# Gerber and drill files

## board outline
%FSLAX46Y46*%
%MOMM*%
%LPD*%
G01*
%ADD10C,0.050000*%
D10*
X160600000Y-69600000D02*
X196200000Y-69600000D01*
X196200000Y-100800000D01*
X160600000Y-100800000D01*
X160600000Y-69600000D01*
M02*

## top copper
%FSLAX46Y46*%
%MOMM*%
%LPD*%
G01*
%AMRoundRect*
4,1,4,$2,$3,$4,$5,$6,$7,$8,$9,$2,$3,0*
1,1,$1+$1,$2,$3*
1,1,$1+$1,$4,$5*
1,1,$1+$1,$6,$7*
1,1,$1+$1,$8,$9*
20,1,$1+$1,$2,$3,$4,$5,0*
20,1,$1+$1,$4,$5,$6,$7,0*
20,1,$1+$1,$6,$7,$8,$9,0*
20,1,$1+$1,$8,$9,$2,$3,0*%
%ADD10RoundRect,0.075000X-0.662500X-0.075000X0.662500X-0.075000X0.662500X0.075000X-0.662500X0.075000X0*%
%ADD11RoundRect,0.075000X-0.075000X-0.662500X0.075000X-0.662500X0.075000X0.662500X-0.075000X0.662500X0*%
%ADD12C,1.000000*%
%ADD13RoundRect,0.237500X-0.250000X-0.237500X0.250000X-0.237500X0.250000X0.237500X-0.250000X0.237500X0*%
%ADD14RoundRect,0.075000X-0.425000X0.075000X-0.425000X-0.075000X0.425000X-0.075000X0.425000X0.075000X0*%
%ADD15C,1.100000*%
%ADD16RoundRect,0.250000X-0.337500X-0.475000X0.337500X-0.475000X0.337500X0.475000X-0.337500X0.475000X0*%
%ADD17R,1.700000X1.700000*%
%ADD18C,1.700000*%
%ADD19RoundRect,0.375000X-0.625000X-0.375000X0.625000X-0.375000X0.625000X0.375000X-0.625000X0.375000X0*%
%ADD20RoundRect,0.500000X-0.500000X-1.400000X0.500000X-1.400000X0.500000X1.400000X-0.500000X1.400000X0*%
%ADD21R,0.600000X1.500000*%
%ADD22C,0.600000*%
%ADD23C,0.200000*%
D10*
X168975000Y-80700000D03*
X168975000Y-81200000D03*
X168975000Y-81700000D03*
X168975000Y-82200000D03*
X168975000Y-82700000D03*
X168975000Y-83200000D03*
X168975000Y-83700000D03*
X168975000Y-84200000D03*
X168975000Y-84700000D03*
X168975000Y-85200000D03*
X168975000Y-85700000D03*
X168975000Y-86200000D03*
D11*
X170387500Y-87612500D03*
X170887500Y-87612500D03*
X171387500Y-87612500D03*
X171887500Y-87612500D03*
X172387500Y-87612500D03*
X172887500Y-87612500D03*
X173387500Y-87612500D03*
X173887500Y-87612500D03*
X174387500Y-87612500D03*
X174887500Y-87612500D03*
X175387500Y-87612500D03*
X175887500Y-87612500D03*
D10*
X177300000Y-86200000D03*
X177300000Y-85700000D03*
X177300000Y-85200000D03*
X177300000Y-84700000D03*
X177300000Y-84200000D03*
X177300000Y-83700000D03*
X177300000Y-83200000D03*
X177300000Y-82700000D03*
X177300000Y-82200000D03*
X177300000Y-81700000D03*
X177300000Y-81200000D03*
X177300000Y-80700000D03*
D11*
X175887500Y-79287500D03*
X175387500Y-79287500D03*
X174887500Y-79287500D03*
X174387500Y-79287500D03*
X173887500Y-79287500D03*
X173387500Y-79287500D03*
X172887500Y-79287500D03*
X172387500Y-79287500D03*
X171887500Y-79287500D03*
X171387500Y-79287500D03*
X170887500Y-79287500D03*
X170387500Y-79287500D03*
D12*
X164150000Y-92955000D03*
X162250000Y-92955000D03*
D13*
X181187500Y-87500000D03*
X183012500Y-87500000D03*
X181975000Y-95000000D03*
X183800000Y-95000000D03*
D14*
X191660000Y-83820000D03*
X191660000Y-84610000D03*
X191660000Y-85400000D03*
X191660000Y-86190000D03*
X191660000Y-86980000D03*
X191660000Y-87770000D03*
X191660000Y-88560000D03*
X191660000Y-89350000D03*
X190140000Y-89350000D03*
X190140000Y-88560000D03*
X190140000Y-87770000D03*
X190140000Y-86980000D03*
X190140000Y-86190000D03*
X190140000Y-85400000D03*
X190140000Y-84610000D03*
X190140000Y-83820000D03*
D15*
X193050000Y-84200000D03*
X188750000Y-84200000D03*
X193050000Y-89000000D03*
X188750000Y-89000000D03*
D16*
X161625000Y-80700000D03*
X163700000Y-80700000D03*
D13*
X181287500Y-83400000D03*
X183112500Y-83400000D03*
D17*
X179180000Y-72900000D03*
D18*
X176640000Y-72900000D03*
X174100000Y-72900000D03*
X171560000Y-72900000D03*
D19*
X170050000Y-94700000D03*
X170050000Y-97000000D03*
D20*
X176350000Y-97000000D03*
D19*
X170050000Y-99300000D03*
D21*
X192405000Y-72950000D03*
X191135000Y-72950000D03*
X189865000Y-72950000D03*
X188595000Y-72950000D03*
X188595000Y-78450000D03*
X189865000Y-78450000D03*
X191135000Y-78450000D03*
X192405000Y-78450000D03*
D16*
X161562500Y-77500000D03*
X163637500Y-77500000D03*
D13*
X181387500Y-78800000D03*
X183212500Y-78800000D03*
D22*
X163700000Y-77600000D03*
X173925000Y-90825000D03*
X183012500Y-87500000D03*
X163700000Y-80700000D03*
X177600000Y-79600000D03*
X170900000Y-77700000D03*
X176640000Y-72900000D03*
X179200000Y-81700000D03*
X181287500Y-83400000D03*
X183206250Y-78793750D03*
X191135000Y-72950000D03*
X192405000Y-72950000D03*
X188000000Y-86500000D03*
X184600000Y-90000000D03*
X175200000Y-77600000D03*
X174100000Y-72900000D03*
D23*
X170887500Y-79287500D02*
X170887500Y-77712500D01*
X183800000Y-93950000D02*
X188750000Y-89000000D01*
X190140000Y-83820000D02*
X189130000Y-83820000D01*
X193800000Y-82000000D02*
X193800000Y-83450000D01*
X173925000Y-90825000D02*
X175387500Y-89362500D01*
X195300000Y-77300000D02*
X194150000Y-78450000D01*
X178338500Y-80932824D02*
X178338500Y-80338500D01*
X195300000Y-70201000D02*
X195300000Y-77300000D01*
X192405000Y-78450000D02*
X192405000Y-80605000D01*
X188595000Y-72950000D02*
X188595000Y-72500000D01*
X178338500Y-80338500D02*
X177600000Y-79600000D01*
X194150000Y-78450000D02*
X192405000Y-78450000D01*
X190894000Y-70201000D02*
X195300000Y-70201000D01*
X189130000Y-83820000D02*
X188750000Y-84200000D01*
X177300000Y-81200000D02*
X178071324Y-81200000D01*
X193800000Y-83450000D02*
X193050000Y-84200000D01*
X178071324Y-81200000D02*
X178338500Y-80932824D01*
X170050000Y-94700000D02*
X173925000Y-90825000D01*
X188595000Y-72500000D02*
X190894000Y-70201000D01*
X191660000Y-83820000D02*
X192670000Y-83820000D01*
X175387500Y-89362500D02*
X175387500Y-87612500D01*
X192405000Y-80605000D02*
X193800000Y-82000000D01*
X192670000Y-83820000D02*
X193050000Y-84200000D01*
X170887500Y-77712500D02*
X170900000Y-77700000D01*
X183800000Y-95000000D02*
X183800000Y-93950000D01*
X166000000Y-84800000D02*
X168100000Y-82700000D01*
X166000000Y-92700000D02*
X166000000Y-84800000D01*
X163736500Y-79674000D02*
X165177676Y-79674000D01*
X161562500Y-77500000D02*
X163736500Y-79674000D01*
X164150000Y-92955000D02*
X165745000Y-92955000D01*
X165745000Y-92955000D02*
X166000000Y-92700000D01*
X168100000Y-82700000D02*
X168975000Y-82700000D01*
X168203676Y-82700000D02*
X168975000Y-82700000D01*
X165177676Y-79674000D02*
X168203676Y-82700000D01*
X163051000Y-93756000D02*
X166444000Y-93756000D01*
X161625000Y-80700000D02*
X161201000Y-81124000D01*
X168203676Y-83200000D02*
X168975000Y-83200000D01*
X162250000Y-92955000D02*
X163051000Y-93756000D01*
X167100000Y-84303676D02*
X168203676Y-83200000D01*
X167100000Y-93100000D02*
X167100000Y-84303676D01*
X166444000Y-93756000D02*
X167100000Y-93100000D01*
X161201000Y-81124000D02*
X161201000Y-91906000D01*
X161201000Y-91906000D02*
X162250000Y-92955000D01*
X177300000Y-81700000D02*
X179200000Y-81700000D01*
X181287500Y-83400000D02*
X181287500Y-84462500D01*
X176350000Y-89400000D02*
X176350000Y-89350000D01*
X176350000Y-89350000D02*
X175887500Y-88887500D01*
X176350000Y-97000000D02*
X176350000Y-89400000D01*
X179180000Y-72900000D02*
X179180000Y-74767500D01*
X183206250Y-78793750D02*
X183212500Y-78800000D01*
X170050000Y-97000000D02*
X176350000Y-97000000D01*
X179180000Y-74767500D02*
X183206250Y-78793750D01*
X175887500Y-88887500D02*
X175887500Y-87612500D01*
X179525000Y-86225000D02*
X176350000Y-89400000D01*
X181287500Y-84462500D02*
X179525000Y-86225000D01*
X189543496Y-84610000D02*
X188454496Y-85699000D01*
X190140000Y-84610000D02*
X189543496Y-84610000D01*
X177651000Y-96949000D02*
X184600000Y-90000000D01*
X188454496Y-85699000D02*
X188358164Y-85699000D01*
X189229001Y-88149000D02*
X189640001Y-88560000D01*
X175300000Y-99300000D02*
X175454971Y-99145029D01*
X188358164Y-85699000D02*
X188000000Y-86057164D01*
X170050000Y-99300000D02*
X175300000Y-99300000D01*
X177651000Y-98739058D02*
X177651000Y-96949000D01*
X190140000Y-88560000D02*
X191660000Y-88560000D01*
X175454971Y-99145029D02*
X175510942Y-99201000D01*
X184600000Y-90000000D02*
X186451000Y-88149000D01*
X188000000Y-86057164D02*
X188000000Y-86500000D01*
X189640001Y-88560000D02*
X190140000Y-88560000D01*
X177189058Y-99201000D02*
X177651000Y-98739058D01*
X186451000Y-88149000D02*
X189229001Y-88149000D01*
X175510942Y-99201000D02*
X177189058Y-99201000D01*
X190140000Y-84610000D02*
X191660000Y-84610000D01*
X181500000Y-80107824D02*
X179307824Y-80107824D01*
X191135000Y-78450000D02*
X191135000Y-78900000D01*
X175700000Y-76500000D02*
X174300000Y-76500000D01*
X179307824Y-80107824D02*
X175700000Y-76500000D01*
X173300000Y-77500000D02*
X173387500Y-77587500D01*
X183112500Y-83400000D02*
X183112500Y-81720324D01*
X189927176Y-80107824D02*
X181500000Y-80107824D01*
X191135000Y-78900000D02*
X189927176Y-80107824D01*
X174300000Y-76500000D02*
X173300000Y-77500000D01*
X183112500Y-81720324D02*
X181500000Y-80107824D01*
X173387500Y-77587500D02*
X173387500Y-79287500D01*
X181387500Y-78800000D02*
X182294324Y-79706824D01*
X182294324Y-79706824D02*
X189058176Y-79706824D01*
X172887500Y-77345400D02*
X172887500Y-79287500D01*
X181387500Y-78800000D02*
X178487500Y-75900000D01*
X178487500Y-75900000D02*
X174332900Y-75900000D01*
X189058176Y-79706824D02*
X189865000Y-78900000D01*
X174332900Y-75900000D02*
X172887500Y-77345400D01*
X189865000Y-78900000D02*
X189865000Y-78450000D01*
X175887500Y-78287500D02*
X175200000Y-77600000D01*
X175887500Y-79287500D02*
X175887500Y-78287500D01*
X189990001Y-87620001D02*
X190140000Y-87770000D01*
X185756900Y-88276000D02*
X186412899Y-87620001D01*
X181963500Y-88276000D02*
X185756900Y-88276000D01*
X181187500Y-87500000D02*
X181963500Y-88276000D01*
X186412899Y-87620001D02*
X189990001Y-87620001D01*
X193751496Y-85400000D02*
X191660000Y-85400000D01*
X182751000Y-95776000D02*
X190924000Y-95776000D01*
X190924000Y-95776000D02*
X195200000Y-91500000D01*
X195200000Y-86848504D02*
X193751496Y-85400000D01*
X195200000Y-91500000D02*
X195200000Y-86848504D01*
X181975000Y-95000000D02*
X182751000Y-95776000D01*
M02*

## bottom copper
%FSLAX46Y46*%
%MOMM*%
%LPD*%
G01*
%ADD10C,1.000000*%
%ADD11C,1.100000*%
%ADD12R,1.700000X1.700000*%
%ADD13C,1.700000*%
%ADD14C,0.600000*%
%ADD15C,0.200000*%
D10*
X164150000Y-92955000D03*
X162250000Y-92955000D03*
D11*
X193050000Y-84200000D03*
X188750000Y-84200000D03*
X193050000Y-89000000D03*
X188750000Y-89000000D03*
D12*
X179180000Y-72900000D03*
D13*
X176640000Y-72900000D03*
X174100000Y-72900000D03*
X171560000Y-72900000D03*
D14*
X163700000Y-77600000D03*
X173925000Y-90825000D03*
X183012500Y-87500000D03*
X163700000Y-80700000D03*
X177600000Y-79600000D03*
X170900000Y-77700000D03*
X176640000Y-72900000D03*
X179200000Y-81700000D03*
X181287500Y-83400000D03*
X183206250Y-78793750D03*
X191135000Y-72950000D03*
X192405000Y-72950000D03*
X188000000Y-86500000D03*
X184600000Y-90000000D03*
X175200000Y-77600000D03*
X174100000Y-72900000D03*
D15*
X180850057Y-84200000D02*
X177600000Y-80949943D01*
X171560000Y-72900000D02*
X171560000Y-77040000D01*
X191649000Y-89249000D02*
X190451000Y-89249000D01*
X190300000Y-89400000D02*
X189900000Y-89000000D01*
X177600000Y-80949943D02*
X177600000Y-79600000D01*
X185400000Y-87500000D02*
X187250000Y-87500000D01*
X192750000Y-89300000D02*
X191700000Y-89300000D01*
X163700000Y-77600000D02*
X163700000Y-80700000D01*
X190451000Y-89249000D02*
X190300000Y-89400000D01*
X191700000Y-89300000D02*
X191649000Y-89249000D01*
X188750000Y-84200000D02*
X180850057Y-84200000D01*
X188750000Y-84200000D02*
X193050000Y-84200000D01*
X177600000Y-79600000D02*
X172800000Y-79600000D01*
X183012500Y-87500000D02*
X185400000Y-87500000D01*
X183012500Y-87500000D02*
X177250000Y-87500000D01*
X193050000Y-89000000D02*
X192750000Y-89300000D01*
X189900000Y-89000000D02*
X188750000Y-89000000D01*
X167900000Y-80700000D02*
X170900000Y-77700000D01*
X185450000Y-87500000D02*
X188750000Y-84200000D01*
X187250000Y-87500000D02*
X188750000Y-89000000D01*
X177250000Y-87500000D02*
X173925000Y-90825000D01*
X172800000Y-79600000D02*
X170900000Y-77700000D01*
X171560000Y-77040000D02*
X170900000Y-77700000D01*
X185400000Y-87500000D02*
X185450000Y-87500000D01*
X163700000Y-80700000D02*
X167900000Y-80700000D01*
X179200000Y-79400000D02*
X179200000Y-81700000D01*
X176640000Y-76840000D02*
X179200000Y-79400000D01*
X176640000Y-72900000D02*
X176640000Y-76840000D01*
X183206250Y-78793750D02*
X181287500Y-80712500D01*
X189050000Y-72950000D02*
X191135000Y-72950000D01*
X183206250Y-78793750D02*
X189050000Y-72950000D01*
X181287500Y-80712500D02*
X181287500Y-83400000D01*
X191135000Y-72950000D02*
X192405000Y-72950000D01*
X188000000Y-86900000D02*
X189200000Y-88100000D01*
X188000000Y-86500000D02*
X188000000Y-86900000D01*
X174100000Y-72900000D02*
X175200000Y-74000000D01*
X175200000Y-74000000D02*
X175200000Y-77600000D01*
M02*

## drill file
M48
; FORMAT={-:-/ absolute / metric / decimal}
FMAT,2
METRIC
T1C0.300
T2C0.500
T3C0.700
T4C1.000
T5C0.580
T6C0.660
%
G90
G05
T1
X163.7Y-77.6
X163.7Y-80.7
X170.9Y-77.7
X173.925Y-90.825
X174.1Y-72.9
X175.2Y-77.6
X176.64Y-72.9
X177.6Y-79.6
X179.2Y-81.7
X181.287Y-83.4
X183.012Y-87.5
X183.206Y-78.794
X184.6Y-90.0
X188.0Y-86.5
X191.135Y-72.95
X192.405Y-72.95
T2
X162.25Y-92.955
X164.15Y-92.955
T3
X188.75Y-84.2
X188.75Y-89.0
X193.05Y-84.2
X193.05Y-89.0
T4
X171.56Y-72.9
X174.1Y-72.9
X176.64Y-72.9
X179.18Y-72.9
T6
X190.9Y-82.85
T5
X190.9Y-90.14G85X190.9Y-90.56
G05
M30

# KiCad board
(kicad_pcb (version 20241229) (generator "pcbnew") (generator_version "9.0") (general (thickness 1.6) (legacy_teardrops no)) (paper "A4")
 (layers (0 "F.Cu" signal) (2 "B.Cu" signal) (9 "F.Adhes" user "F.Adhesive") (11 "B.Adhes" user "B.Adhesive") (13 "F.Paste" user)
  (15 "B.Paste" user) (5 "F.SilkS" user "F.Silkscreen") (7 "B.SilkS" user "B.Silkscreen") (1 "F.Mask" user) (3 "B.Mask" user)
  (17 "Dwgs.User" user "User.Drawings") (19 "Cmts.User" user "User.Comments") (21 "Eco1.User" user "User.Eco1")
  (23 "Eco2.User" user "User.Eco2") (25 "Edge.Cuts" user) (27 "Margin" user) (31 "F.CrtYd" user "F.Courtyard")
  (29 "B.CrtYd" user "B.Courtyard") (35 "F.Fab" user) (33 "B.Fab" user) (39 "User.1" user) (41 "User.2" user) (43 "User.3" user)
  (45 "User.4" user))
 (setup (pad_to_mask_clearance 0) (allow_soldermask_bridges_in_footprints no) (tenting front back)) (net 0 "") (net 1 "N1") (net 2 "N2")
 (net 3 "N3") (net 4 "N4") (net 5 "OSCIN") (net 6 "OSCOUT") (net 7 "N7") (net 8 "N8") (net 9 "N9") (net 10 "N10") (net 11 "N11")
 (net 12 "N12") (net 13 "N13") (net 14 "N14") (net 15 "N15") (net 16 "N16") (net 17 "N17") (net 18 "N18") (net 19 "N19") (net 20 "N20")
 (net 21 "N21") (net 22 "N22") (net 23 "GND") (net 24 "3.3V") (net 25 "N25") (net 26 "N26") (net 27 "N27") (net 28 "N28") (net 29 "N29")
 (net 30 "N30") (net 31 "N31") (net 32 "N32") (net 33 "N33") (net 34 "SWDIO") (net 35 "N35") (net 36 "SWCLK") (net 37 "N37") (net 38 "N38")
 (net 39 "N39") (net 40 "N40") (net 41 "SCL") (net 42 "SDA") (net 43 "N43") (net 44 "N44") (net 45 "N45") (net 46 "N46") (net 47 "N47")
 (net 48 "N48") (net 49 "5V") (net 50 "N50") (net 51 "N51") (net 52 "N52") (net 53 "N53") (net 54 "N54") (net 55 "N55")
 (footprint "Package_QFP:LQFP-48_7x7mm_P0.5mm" (layer "F.Cu") (at 173.1375 83.45)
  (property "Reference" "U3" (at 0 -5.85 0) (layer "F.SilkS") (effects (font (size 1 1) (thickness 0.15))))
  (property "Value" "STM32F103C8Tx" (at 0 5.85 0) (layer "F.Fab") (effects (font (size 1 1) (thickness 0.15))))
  (pad "1" smd roundrect (at -4.1625 -2.75) (size 1.475 0.3) (layers "F.Cu" "F.Mask" "F.Paste") (roundrect_rratio 0.25) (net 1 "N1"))
  (pad "2" smd roundrect (at -4.1625 -2.25) (size 1.475 0.3) (layers "F.Cu" "F.Mask" "F.Paste") (roundrect_rratio 0.25) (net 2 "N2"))
  (pad "3" smd roundrect (at -4.1625 -1.75) (size 1.475 0.3) (layers "F.Cu" "F.Mask" "F.Paste") (roundrect_rratio 0.25) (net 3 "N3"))
  (pad "4" smd roundrect (at -4.1625 -1.25) (size 1.475 0.3) (layers "F.Cu" "F.Mask" "F.Paste") (roundrect_rratio 0.25) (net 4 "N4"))
  (pad "5" smd roundrect (at -4.1625 -0.75) (size 1.475 0.3) (layers "F.Cu" "F.Mask" "F.Paste") (roundrect_rratio 0.25) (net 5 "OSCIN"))
  (pad "6" smd roundrect (at -4.1625 -0.25) (size 1.475 0.3) (layers "F.Cu" "F.Mask" "F.Paste") (roundrect_rratio 0.25) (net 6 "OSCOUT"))
  (pad "7" smd roundrect (at -4.1625 0.25) (size 1.475 0.3) (layers "F.Cu" "F.Mask" "F.Paste") (roundrect_rratio 0.25) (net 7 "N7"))
  (pad "8" smd roundrect (at -4.1625 0.75) (size 1.475 0.3) (layers "F.Cu" "F.Mask" "F.Paste") (roundrect_rratio 0.25) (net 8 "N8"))
  (pad "9" smd roundrect (at -4.1625 1.25) (size 1.475 0.3) (layers "F.Cu" "F.Mask" "F.Paste") (roundrect_rratio 0.25) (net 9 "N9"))
  (pad "10" smd roundrect (at -4.1625 1.75) (size 1.475 0.3) (layers "F.Cu" "F.Mask" "F.Paste") (roundrect_rratio 0.25) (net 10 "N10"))
  (pad "11" smd roundrect (at -4.1625 2.25) (size 1.475 0.3) (layers "F.Cu" "F.Mask" "F.Paste") (roundrect_rratio 0.25) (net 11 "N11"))
  (pad "12" smd roundrect (at -4.1625 2.75) (size 1.475 0.3) (layers "F.Cu" "F.Mask" "F.Paste") (roundrect_rratio 0.25) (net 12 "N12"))
  (pad "13" smd roundrect (at -2.75 4.1625) (size 0.3 1.475) (layers "F.Cu" "F.Mask" "F.Paste") (roundrect_rratio 0.25) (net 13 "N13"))
  (pad "14" smd roundrect (at -2.25 4.1625) (size 0.3 1.475) (layers "F.Cu" "F.Mask" "F.Paste") (roundrect_rratio 0.25) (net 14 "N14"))
  (pad "15" smd roundrect (at -1.75 4.1625) (size 0.3 1.475) (layers "F.Cu" "F.Mask" "F.Paste") (roundrect_rratio 0.25) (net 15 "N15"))
  (pad "16" smd roundrect (at -1.25 4.1625) (size 0.3 1.475) (layers "F.Cu" "F.Mask" "F.Paste") (roundrect_rratio 0.25) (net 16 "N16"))
  (pad "17" smd roundrect (at -0.75 4.1625) (size 0.3 1.475) (layers "F.Cu" "F.Mask" "F.Paste") (roundrect_rratio 0.25) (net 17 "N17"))
  (pad "18" smd roundrect (at -0.25 4.1625) (size 0.3 1.475) (layers "F.Cu" "F.Mask" "F.Paste") (roundrect_rratio 0.25) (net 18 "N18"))
  (pad "19" smd roundrect (at 0.25 4.1625) (size 0.3 1.475) (layers "F.Cu" "F.Mask" "F.Paste") (roundrect_rratio 0.25) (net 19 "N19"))
  (pad "20" smd roundrect (at 0.75 4.1625) (size 0.3 1.475) (layers "F.Cu" "F.Mask" "F.Paste") (roundrect_rratio 0.25) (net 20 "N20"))
  (pad "21" smd roundrect (at 1.25 4.1625) (size 0.3 1.475) (layers "F.Cu" "F.Mask" "F.Paste") (roundrect_rratio 0.25) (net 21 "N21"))
  (pad "22" smd roundrect (at 1.75 4.1625) (size 0.3 1.475) (layers "F.Cu" "F.Mask" "F.Paste") (roundrect_rratio 0.25) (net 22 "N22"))
  (pad "23" smd roundrect (at 2.25 4.1625) (size 0.3 1.475) (layers "F.Cu" "F.Mask" "F.Paste") (roundrect_rratio 0.25) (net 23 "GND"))
  (pad "24" smd roundrect (at 2.75 4.1625) (size 0.3 1.475) (layers "F.Cu" "F.Mask" "F.Paste") (roundrect_rratio 0.25) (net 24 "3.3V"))
  (pad "25" smd roundrect (at 4.1625 2.75) (size 1.475 0.3) (layers "F.Cu" "F.Mask" "F.Paste") (roundrect_rratio 0.25) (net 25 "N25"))
  (pad "26" smd roundrect (at 4.1625 2.25) (size 1.475 0.3) (layers "F.Cu" "F.Mask" "F.Paste") (roundrect_rratio 0.25) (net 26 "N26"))
  (pad "27" smd roundrect (at 4.1625 1.75) (size 1.475 0.3) (layers "F.Cu" "F.Mask" "F.Paste") (roundrect_rratio 0.25) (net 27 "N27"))
  (pad "28" smd roundrect (at 4.1625 1.25) (size 1.475 0.3) (layers "F.Cu" "F.Mask" "F.Paste") (roundrect_rratio 0.25) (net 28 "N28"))
  (pad "29" smd roundrect (at 4.1625 0.75) (size 1.475 0.3) (layers "F.Cu" "F.Mask" "F.Paste") (roundrect_rratio 0.25) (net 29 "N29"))
  (pad "30" smd roundrect (at 4.1625 0.25) (size 1.475 0.3) (layers "F.Cu" "F.Mask" "F.Paste") (roundrect_rratio 0.25) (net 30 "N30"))
  (pad "31" smd roundrect (at 4.1625 -0.25) (size 1.475 0.3) (layers "F.Cu" "F.Mask" "F.Paste") (roundrect_rratio 0.25) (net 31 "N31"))
  (pad "32" smd roundrect (at 4.1625 -0.75) (size 1.475 0.3) (layers "F.Cu" "F.Mask" "F.Paste") (roundrect_rratio 0.25) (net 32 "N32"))
  (pad "33" smd roundrect (at 4.1625 -1.25) (size 1.475 0.3) (layers "F.Cu" "F.Mask" "F.Paste") (roundrect_rratio 0.25) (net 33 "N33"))
  (pad "34" smd roundrect (at 4.1625 -1.75) (size 1.475 0.3) (layers "F.Cu" "F.Mask" "F.Paste") (roundrect_rratio 0.25) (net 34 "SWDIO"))
  (pad "35" smd roundrect (at 4.1625 -2.25) (size 1.475 0.3) (layers "F.Cu" "F.Mask" "F.Paste") (roundrect_rratio 0.25) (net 23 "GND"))
  (pad "36" smd roundrect (at 4.1625 -2.75) (size 1.475 0.3) (layers "F.Cu" "F.Mask" "F.Paste") (roundrect_rratio 0.25) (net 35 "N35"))
  (pad "37" smd roundrect (at 2.75 -4.1625) (size 0.3 1.475) (layers "F.Cu" "F.Mask" "F.Paste") (roundrect_rratio 0.25) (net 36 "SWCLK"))
  (pad "38" smd roundrect (at 2.25 -4.1625) (size 0.3 1.475) (layers "F.Cu" "F.Mask" "F.Paste") (roundrect_rratio 0.25) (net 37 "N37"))
  (pad "39" smd roundrect (at 1.75 -4.1625) (size 0.3 1.475) (layers "F.Cu" "F.Mask" "F.Paste") (roundrect_rratio 0.25) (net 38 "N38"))
  (pad "40" smd roundrect (at 1.25 -4.1625) (size 0.3 1.475) (layers "F.Cu" "F.Mask" "F.Paste") (roundrect_rratio 0.25) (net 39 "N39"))
  (pad "41" smd roundrect (at 0.75 -4.1625) (size 0.3 1.475) (layers "F.Cu" "F.Mask" "F.Paste") (roundrect_rratio 0.25) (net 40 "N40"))
  (pad "42" smd roundrect (at 0.25 -4.1625) (size 0.3 1.475) (layers "F.Cu" "F.Mask" "F.Paste") (roundrect_rratio 0.25) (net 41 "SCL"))
  (pad "43" smd roundrect (at -0.25 -4.1625) (size 0.3 1.475) (layers "F.Cu" "F.Mask" "F.Paste") (roundrect_rratio 0.25) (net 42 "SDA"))
  (pad "44" smd roundrect (at -0.75 -4.1625) (size 0.3 1.475) (layers "F.Cu" "F.Mask" "F.Paste") (roundrect_rratio 0.25) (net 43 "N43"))
  (pad "45" smd roundrect (at -1.25 -4.1625) (size 0.3 1.475) (layers "F.Cu" "F.Mask" "F.Paste") (roundrect_rratio 0.25) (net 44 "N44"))
  (pad "46" smd roundrect (at -1.75 -4.1625) (size 0.3 1.475) (layers "F.Cu" "F.Mask" "F.Paste") (roundrect_rratio 0.25) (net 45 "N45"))
  (pad "47" smd roundrect (at -2.25 -4.1625) (size 0.3 1.475) (layers "F.Cu" "F.Mask" "F.Paste") (roundrect_rratio 0.25) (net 23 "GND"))
  (pad "48" smd roundrect (at -2.75 -4.1625) (size 0.3 1.475) (layers "F.Cu" "F.Mask" "F.Paste") (roundrect_rratio 0.25) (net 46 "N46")))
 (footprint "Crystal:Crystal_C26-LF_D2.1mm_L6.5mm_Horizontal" (layer "F.Cu") (at 164.15 92.955 180)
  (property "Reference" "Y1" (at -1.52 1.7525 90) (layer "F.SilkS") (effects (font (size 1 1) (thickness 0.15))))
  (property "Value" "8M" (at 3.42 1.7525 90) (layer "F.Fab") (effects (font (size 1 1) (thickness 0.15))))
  (pad "1" thru_hole circle (at 0 0 180) (size 1 1) (drill 0.5) (layers "*.Cu" "*.Mask") (remove_unused_layers no) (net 5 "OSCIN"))
  (pad "2" thru_hole circle (at 1.9 0 180) (size 1 1) (drill 0.5) (layers "*.Cu" "*.Mask") (remove_unused_layers no) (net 6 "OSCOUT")))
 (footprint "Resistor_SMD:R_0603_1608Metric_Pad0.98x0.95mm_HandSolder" (layer "F.Cu") (at 182.1 87.5)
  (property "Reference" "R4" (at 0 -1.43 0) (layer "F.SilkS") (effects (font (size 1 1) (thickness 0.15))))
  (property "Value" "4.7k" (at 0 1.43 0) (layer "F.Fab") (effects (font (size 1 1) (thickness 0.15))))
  (pad "1" smd roundrect (at -0.9125 0) (size 0.975 0.95) (layers "F.Cu" "F.Mask" "F.Paste") (roundrect_rratio 0.25) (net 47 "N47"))
  (pad "2" smd roundrect (at 0.9125 0) (size 0.975 0.95) (layers "F.Cu" "F.Mask" "F.Paste") (roundrect_rratio 0.25) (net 23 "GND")))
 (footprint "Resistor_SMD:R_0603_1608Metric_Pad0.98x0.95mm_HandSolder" (layer "F.Cu") (at 182.8875 95)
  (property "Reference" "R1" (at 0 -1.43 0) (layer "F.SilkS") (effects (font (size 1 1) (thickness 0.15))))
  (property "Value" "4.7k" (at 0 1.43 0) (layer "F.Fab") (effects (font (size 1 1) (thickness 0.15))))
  (pad "1" smd roundrect (at -0.9125 0) (size 0.975 0.95) (layers "F.Cu" "F.Mask" "F.Paste") (roundrect_rratio 0.25) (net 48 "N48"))
  (pad "2" smd roundrect (at 0.9125 0) (size 0.975 0.95) (layers "F.Cu" "F.Mask" "F.Paste") (roundrect_rratio 0.25) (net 23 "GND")))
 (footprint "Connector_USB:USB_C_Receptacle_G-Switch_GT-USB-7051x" (layer "F.Cu") (at 190.9 86.6 -90)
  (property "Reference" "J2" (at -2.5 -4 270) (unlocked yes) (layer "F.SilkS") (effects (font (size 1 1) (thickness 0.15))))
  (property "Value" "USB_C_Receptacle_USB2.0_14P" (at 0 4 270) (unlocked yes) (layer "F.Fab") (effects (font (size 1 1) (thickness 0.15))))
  (pad "" np_thru_hole circle (at -3.75 0 270) (size 0.66 0.66) (drill 0.66) (layers "*.Cu" "*.Mask"))
  (pad "" np_thru_hole oval (at 3.75 0 270) (size 1 0.58) (drill oval 1 0.58) (layers "*.Cu" "*.Mask"))
  (pad "A1" smd roundrect (at -2.78 -0.76 270) (size 0.3 1) (layers "F.Cu" "F.Mask" "F.Paste") (roundrect_rratio 0.25) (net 23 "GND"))
  (pad "A4" smd roundrect (at -1.99 -0.76 270) (size 0.3 1) (layers "F.Cu" "F.Mask" "F.Paste") (roundrect_rratio 0.25) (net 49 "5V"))
  (pad "A5" smd roundrect (at -1.2 -0.76 270) (size 0.3 1) (layers "F.Cu" "F.Mask" "F.Paste") (roundrect_rratio 0.25) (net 48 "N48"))
  (pad "A6" smd roundrect (at -0.41 -0.76 270) (size 0.3 1) (layers "F.Cu" "F.Mask" "F.Paste") (roundrect_rratio 0.25) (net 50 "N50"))
  (pad "A7" smd roundrect (at 0.38 -0.76 270) (size 0.3 1) (layers "F.Cu" "F.Mask" "F.Paste") (roundrect_rratio 0.25) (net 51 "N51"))
  (pad "A8" smd roundrect (at 1.17 -0.76 270) (size 0.3 1) (layers "F.Cu" "F.Mask" "F.Paste") (roundrect_rratio 0.25))
  (pad "A9" smd roundrect (at 1.96 -0.76 270) (size 0.3 1) (layers "F.Cu" "F.Mask" "F.Paste") (roundrect_rratio 0.25) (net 49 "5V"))
  (pad "A12" smd roundrect (at 2.75 -0.76 270) (size 0.3 1) (layers "F.Cu" "F.Mask" "F.Paste") (roundrect_rratio 0.25) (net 23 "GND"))
  (pad "B1" smd roundrect (at 2.75 0.76 270) (size 0.3 1) (layers "F.Cu" "F.Mask" "F.Paste") (roundrect_rratio 0.25) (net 23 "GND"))
  (pad "B4" smd roundrect (at 1.96 0.76 270) (size 0.3 1) (layers "F.Cu" "F.Mask" "F.Paste") (roundrect_rratio 0.25) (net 49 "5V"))
  (pad "B5" smd roundrect (at 1.17 0.76 270) (size 0.3 1) (layers "F.Cu" "F.Mask" "F.Paste") (roundrect_rratio 0.25) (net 47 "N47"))
  (pad "B6" smd roundrect (at 0.38 0.76 270) (size 0.3 1) (layers "F.Cu" "F.Mask" "F.Paste") (roundrect_rratio 0.25) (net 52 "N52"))
  (pad "B7" smd roundrect (at -0.41 0.76 270) (size 0.3 1) (layers "F.Cu" "F.Mask" "F.Paste") (roundrect_rratio 0.25) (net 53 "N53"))
  (pad "B8" smd roundrect (at -1.2 0.76 270) (size 0.3 1) (layers "F.Cu" "F.Mask" "F.Paste") (roundrect_rratio 0.25))
  (pad "B9" smd roundrect (at -1.99 0.76 270) (size 0.3 1) (layers "F.Cu" "F.Mask" "F.Paste") (roundrect_rratio 0.25) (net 49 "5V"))
  (pad "B12" smd roundrect (at -2.78 0.76 270) (size 0.3 1) (layers "F.Cu" "F.Mask" "F.Paste") (roundrect_rratio 0.25) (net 23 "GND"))
  (pad "S1" thru_hole circle (at -2.4 -2.15 270) (size 1.1 1.1) (drill 0.7) (layers "*.Cu" "*.Mask" "F.Paste") (remove_unused_layers no)
   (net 23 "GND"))
  (pad "S1" thru_hole circle (at -2.4 2.15 270) (size 1.1 1.1) (drill 0.7) (layers "*.Cu" "*.Mask" "F.Paste") (remove_unused_layers no)
   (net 23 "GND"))
  (pad "S1" thru_hole circle (at 2.4 -2.15 270) (size 1.1 1.1) (drill 0.7) (layers "*.Cu" "*.Mask" "F.Paste") (remove_unused_layers no)
   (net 23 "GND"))
  (pad "S1" thru_hole circle (at 2.4 2.15 270) (size 1.1 1.1) (drill 0.7) (layers "*.Cu" "*.Mask" "F.Paste") (remove_unused_layers no)
   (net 23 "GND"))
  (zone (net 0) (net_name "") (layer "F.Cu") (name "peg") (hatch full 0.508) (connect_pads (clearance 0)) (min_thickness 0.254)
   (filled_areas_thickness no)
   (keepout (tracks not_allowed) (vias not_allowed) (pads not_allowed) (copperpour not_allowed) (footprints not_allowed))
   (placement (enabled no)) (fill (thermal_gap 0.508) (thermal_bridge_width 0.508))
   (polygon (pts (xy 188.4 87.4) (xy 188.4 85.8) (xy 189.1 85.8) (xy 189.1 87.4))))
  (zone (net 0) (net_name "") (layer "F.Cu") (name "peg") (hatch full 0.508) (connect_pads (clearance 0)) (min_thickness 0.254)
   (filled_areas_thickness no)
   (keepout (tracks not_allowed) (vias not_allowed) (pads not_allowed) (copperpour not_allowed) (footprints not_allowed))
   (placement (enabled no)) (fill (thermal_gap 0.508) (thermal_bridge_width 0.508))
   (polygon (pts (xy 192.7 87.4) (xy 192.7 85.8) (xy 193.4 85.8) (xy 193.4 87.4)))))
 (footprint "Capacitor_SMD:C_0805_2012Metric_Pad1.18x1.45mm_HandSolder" (layer "F.Cu") (at 162.6625 80.7)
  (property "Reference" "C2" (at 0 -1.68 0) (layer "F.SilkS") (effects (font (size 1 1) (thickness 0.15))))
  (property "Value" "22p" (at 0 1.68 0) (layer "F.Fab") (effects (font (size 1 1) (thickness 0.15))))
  (pad "1" smd roundrect (at -1.0375 0) (size 1.175 1.45) (layers "F.Cu" "F.Mask" "F.Paste") (roundrect_rratio 0.212766) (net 6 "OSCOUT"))
  (pad "2" smd roundrect (at 1.0375 0) (size 1.175 1.45) (layers "F.Cu" "F.Mask" "F.Paste") (roundrect_rratio 0.212766) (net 23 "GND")))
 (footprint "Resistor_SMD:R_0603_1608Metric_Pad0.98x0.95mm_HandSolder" (layer "F.Cu") (at 182.2 83.4)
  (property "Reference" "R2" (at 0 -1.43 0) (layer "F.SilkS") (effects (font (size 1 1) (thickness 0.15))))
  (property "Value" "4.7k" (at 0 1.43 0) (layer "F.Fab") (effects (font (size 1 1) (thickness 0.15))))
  (pad "1" smd roundrect (at -0.9125 0) (size 0.975 0.95) (layers "F.Cu" "F.Mask" "F.Paste") (roundrect_rratio 0.25) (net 24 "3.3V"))
  (pad "2" smd roundrect (at 0.9125 0) (size 0.975 0.95) (layers "F.Cu" "F.Mask" "F.Paste") (roundrect_rratio 0.25) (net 41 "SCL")))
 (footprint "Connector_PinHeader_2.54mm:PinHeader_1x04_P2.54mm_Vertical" (layer "F.Cu") (at 179.18 72.9 -90)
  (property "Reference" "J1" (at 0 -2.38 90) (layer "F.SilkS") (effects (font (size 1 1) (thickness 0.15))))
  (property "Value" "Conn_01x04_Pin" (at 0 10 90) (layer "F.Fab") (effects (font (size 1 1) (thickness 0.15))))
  (pad "1" thru_hole rect (at 0 0 270) (size 1.7 1.7) (drill 1) (layers "*.Cu" "*.Mask") (remove_unused_layers no) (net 24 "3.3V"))
  (pad "2" thru_hole circle (at 0 2.54 270) (size 1.7 1.7) (drill 1) (layers "*.Cu" "*.Mask") (remove_unused_layers no) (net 34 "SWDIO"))
  (pad "3" thru_hole circle (at 0 5.08 270) (size 1.7 1.7) (drill 1) (layers "*.Cu" "*.Mask") (remove_unused_layers no) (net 36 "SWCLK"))
  (pad "4" thru_hole circle (at 0 7.62 270) (size 1.7 1.7) (drill 1) (layers "*.Cu" "*.Mask") (remove_unused_layers no) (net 23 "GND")))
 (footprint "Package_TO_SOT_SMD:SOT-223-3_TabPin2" (layer "F.Cu") (at 173.2 97)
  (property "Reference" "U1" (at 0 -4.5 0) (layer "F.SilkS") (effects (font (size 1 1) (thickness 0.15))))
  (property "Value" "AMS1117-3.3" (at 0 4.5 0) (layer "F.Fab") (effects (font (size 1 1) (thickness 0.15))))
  (pad "1" smd roundrect (at -3.15 -2.3) (size 2 1.5) (layers "F.Cu" "F.Mask" "F.Paste") (roundrect_rratio 0.25) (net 23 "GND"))
  (pad "2" smd roundrect (at -3.15 0) (size 2 1.5) (layers "F.Cu" "F.Mask" "F.Paste") (roundrect_rratio 0.25) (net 24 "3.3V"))
  (pad "2" smd roundrect (at 3.15 0) (size 2 3.8) (layers "F.Cu" "F.Mask" "F.Paste") (roundrect_rratio 0.25) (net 24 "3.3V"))
  (pad "3" smd roundrect (at -3.15 2.3) (size 2 1.5) (layers "F.Cu" "F.Mask" "F.Paste") (roundrect_rratio 0.25) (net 49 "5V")))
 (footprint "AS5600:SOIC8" (layer "F.Cu") (at 190.5 75.7 180)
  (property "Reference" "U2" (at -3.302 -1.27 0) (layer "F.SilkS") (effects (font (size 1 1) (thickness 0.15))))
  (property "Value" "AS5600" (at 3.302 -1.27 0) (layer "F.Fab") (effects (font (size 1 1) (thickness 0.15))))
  (pad "1" smd rect (at -1.905 2.75 180) (size 0.6 1.5) (layers "F.Cu" "F.Mask" "F.Paste") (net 24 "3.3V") (solder_mask_margin 0.102))
  (pad "2" smd rect (at -0.635 2.75 180) (size 0.6 1.5) (layers "F.Cu" "F.Mask" "F.Paste") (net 24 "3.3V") (solder_mask_margin 0.102))
  (pad "3" smd rect (at 0.635 2.75 180) (size 0.6 1.5) (layers "F.Cu" "F.Mask" "F.Paste") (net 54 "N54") (solder_mask_margin 0.102))
  (pad "4" smd rect (at 1.905 2.75 180) (size 0.6 1.5) (layers "F.Cu" "F.Mask" "F.Paste") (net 23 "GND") (solder_mask_margin 0.102))
  (pad "5" smd rect (at 1.905 -2.75 180) (size 0.6 1.5) (layers "F.Cu" "F.Mask" "F.Paste") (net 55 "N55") (solder_mask_margin 0.102))
  (pad "6" smd rect (at 0.635 -2.75 180) (size 0.6 1.5) (layers "F.Cu" "F.Mask" "F.Paste") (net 42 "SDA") (solder_mask_margin 0.102))
  (pad "7" smd rect (at -0.635 -2.75 180) (size 0.6 1.5) (layers "F.Cu" "F.Mask" "F.Paste") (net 41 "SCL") (solder_mask_margin 0.102))
  (pad "8" smd rect (at -1.905 -2.75 180) (size 0.6 1.5) (layers "F.Cu" "F.Mask" "F.Paste") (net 23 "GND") (solder_mask_margin 0.102)))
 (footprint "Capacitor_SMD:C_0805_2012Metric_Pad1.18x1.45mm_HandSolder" (layer "F.Cu") (at 162.6 77.5)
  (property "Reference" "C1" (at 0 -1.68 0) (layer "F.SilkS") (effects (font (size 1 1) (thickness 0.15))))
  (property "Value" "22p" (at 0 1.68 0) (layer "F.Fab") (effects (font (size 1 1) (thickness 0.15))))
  (pad "1" smd roundrect (at -1.0375 0) (size 1.175 1.45) (layers "F.Cu" "F.Mask" "F.Paste") (roundrect_rratio 0.212766) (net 5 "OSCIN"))
  (pad "2" smd roundrect (at 1.0375 0) (size 1.175 1.45) (layers "F.Cu" "F.Mask" "F.Paste") (roundrect_rratio 0.212766) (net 23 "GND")))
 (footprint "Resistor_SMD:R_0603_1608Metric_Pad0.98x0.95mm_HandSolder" (layer "F.Cu") (at 182.3 78.8)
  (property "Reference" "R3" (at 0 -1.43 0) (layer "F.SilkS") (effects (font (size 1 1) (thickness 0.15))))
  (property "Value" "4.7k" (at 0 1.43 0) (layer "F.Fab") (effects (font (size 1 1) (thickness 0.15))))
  (pad "1" smd roundrect (at -0.9125 0) (size 0.975 0.95) (layers "F.Cu" "F.Mask" "F.Paste") (roundrect_rratio 0.25) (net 42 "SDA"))
  (pad "2" smd roundrect (at 0.9125 0) (size 0.975 0.95) (layers "F.Cu" "F.Mask" "F.Paste") (roundrect_rratio 0.25) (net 24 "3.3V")))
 (gr_rect (start 160.6 69.6) (end 196.2 100.8) (stroke (width 0.05) (type default)) (fill no) (layer "Edge.Cuts"))
 (segment (start 170.8875 79.2875) (end 170.8875 77.7125) (width 0.2) (layer "F.Cu") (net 23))
 (segment (start 183.8 93.95) (end 188.75 89) (width 0.2) (layer "F.Cu") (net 23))
 (segment (start 190.14 83.82) (end 189.13 83.82) (width 0.2) (layer "F.Cu") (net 23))
 (segment (start 193.8 82) (end 193.8 83.45) (width 0.2) (layer "F.Cu") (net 23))
 (segment (start 173.925 90.825) (end 175.3875 89.3625) (width 0.2) (layer "F.Cu") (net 23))
 (segment (start 195.3 77.3) (end 194.15 78.45) (width 0.2) (layer "F.Cu") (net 23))
 (segment (start 178.3385 80.932824) (end 178.3385 80.3385) (width 0.2) (layer "F.Cu") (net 23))
 (segment (start 195.3 70.201) (end 195.3 77.3) (width 0.2) (layer "F.Cu") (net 23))
 (segment (start 192.405 78.45) (end 192.405 80.605) (width 0.2) (layer "F.Cu") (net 23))
 (segment (start 188.595 72.95) (end 188.595 72.5) (width 0.2) (layer "F.Cu") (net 23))
 (segment (start 178.3385 80.3385) (end 177.6 79.6) (width 0.2) (layer "F.Cu") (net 23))
 (segment (start 194.15 78.45) (end 192.405 78.45) (width 0.2) (layer "F.Cu") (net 23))
 (segment (start 190.894 70.201) (end 195.3 70.201) (width 0.2) (layer "F.Cu") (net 23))
 (segment (start 189.13 83.82) (end 188.75 84.2) (width 0.2) (layer "F.Cu") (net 23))
 (segment (start 177.3 81.2) (end 178.071324 81.2) (width 0.2) (layer "F.Cu") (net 23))
 (segment (start 193.8 83.45) (end 193.05 84.2) (width 0.2) (layer "F.Cu") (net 23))
 (segment (start 178.071324 81.2) (end 178.3385 80.932824) (width 0.2) (layer "F.Cu") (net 23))
 (segment (start 170.05 94.7) (end 173.925 90.825) (width 0.2) (layer "F.Cu") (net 23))
 (segment (start 188.595 72.5) (end 190.894 70.201) (width 0.2) (layer "F.Cu") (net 23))
 (segment (start 191.66 83.82) (end 192.67 83.82) (width 0.2) (layer "F.Cu") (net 23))
 (segment (start 175.3875 89.3625) (end 175.3875 87.6125) (width 0.2) (layer "F.Cu") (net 23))
 (segment (start 192.405 80.605) (end 193.8 82) (width 0.2) (layer "F.Cu") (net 23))
 (segment (start 192.67 83.82) (end 193.05 84.2) (width 0.2) (layer "F.Cu") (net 23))
 (segment (start 170.8875 77.7125) (end 170.9 77.7) (width 0.2) (layer "F.Cu") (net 23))
 (segment (start 183.8 95) (end 183.8 93.95) (width 0.2) (layer "F.Cu") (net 23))
 (via (at 163.7 77.6) (size 0.6) (drill 0.3) (layers "F.Cu" "B.Cu") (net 23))
 (via (at 173.925 90.825) (size 0.6) (drill 0.3) (layers "F.Cu" "B.Cu") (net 23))
 (via (at 183.0125 87.5) (size 0.6) (drill 0.3) (layers "F.Cu" "B.Cu") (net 23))
 (via (at 163.7 80.7) (size 0.6) (drill 0.3) (layers "F.Cu" "B.Cu") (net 23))
 (via (at 177.6 79.6) (size 0.6) (drill 0.3) (layers "F.Cu" "B.Cu") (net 23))
 (via (at 170.9 77.7) (size 0.6) (drill 0.3) (layers "F.Cu" "B.Cu") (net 23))
 (segment (start 180.850057 84.2) (end 177.6 80.949943) (width 0.2) (layer "B.Cu") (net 23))
 (segment (start 171.56 72.9) (end 171.56 77.04) (width 0.2) (layer "B.Cu") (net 23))
 (segment (start 191.649 89.249) (end 190.451 89.249) (width 0.2) (layer "B.Cu") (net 23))
 (segment (start 190.3 89.4) (end 189.9 89) (width 0.2) (layer "B.Cu") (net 23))
 (segment (start 177.6 80.949943) (end 177.6 79.6) (width 0.2) (layer "B.Cu") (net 23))
 (segment (start 185.4 87.5) (end 187.25 87.5) (width 0.2) (layer "B.Cu") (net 23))
 (segment (start 192.75 89.3) (end 191.7 89.3) (width 0.2) (layer "B.Cu") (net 23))
 (segment (start 163.7 77.6) (end 163.7 80.7) (width 0.2) (layer "B.Cu") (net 23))
 (segment (start 190.451 89.249) (end 190.3 89.4) (width 0.2) (layer "B.Cu") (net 23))
 (segment (start 191.7 89.3) (end 191.649 89.249) (width 0.2) (layer "B.Cu") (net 23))
 (segment (start 188.75 84.2) (end 180.850057 84.2) (width 0.2) (layer "B.Cu") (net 23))
 (segment (start 188.75 84.2) (end 193.05 84.2) (width 0.2) (layer "B.Cu") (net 23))
 (segment (start 177.6 79.6) (end 172.8 79.6) (width 0.2) (layer "B.Cu") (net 23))
 (segment (start 183.0125 87.5) (end 185.4 87.5) (width 0.2) (layer "B.Cu") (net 23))
 (segment (start 183.0125 87.5) (end 177.25 87.5) (width 0.2) (layer "B.Cu") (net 23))
 (segment (start 193.05 89) (end 192.75 89.3) (width 0.2) (layer "B.Cu") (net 23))
 (segment (start 189.9 89) (end 188.75 89) (width 0.2) (layer "B.Cu") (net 23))
 (segment (start 167.9 80.7) (end 170.9 77.7) (width 0.2) (layer "B.Cu") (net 23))
 (segment (start 185.45 87.5) (end 188.75 84.2) (width 0.2) (layer "B.Cu") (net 23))
 (segment (start 187.25 87.5) (end 188.75 89) (width 0.2) (layer "B.Cu") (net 23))
 (segment (start 177.25 87.5) (end 173.925 90.825) (width 0.2) (layer "B.Cu") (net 23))
 (segment (start 172.8 79.6) (end 170.9 77.7) (width 0.2) (layer "B.Cu") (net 23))
 (segment (start 171.56 77.04) (end 170.9 77.7) (width 0.2) (layer "B.Cu") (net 23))
 (segment (start 185.4 87.5) (end 185.45 87.5) (width 0.2) (layer "B.Cu") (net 23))
 (segment (start 163.7 80.7) (end 167.9 80.7) (width 0.2) (layer "B.Cu") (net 23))
 (segment (start 166 84.8) (end 168.1 82.7) (width 0.2) (layer "F.Cu") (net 5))
 (segment (start 166 92.7) (end 166 84.8) (width 0.2) (layer "F.Cu") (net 5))
 (segment (start 163.7365 79.674) (end 165.177676 79.674) (width 0.2) (layer "F.Cu") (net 5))
 (segment (start 161.5625 77.5) (end 163.7365 79.674) (width 0.2) (layer "F.Cu") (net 5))
 (segment (start 164.15 92.955) (end 165.745 92.955) (width 0.2) (layer "F.Cu") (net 5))
 (segment (start 165.745 92.955) (end 166 92.7) (width 0.2) (layer "F.Cu") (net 5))
 (segment (start 168.1 82.7) (end 168.975 82.7) (width 0.2) (layer "F.Cu") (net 5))
 (segment (start 168.203676 82.7) (end 168.975 82.7) (width 0.2) (layer "F.Cu") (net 5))
 (segment (start 165.177676 79.674) (end 168.203676 82.7) (width 0.2) (layer "F.Cu") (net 5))
 (segment (start 163.051 93.756) (end 166.444 93.756) (width 0.2) (layer "F.Cu") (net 6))
 (segment (start 161.625 80.7) (end 161.201 81.124) (width 0.2) (layer "F.Cu") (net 6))
 (segment (start 168.203676 83.2) (end 168.975 83.2) (width 0.2) (layer "F.Cu") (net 6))
 (segment (start 162.25 92.955) (end 163.051 93.756) (width 0.2) (layer "F.Cu") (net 6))
 (segment (start 167.1 84.303676) (end 168.203676 83.2) (width 0.2) (layer "F.Cu") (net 6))
 (segment (start 167.1 93.1) (end 167.1 84.303676) (width 0.2) (layer "F.Cu") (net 6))
 (segment (start 166.444 93.756) (end 167.1 93.1) (width 0.2) (layer "F.Cu") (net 6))
 (segment (start 161.201 81.124) (end 161.201 91.906) (width 0.2) (layer "F.Cu") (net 6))
 (segment (start 161.201 91.906) (end 162.25 92.955) (width 0.2) (layer "F.Cu") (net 6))
 (segment (start 177.3 81.7) (end 179.2 81.7) (width 0.2) (layer "F.Cu") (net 34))
 (via (at 176.64 72.9) (size 0.6) (drill 0.3) (layers "F.Cu" "B.Cu") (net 34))
 (via (at 179.2 81.7) (size 0.6) (drill 0.3) (layers "F.Cu" "B.Cu") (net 34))
 (segment (start 179.2 79.4) (end 179.2 81.7) (width 0.2) (layer "B.Cu") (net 34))
 (segment (start 176.64 76.84) (end 179.2 79.4) (width 0.2) (layer "B.Cu") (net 34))
 (segment (start 176.64 72.9) (end 176.64 76.84) (width 0.2) (layer "B.Cu") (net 34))
 (segment (start 181.2875 83.4) (end 181.2875 84.4625) (width 0.2) (layer "F.Cu") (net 24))
 (segment (start 176.35 89.4) (end 176.35 89.35) (width 0.2) (layer "F.Cu") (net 24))
 (segment (start 176.35 89.35) (end 175.8875 88.8875) (width 0.2) (layer "F.Cu") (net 24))
 (segment (start 176.35 97) (end 176.35 89.4) (width 0.2) (layer "F.Cu") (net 24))
 (segment (start 179.18 72.9) (end 179.18 74.7675) (width 0.2) (layer "F.Cu") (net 24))
 (segment (start 183.20625 78.79375) (end 183.2125 78.8) (width 0.2) (layer "F.Cu") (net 24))
 (segment (start 170.05 97) (end 176.35 97) (width 0.2) (layer "F.Cu") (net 24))
 (segment (start 179.18 74.7675) (end 183.20625 78.79375) (width 0.2) (layer "F.Cu") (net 24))
 (segment (start 175.8875 88.8875) (end 175.8875 87.6125) (width 0.2) (layer "F.Cu") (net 24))
 (segment (start 179.525 86.225) (end 176.35 89.4) (width 0.2) (layer "F.Cu") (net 24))
 (segment (start 181.2875 84.4625) (end 179.525 86.225) (width 0.2) (layer "F.Cu") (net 24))
 (via (at 181.2875 83.4) (size 0.6) (drill 0.3) (layers "F.Cu" "B.Cu") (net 24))
 (via (at 183.20625 78.79375) (size 0.6) (drill 0.3) (layers "F.Cu" "B.Cu") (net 24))
 (via (at 191.135 72.95) (size 0.6) (drill 0.3) (layers "F.Cu" "B.Cu") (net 24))
 (via (at 192.405 72.95) (size 0.6) (drill 0.3) (layers "F.Cu" "B.Cu") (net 24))
 (segment (start 183.20625 78.79375) (end 181.2875 80.7125) (width 0.2) (layer "B.Cu") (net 24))
 (segment (start 189.05 72.95) (end 191.135 72.95) (width 0.2) (layer "B.Cu") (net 24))
 (segment (start 183.20625 78.79375) (end 189.05 72.95) (width 0.2) (layer "B.Cu") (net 24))
 (segment (start 181.2875 80.7125) (end 181.2875 83.4) (width 0.2) (layer "B.Cu") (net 24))
 (segment (start 191.135 72.95) (end 192.405 72.95) (width 0.2) (layer "B.Cu") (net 24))
 (segment (start 189.543496 84.61) (end 188.454496 85.699) (width 0.2) (layer "F.Cu") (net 49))
 (segment (start 190.14 84.61) (end 189.543496 84.61) (width 0.2) (layer "F.Cu") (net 49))
 (segment (start 177.651 96.949) (end 184.6 90) (width 0.2) (layer "F.Cu") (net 49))
 (segment (start 188.454496 85.699) (end 188.358164 85.699) (width 0.2) (layer "F.Cu") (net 49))
 (segment (start 189.229001 88.149) (end 189.640001 88.56) (width 0.2) (layer "F.Cu") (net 49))
 (segment (start 175.3 99.3) (end 175.454971 99.145029) (width 0.2) (layer "F.Cu") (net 49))
 (segment (start 188.358164 85.699) (end 188 86.057164) (width 0.2) (layer "F.Cu") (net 49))
 (segment (start 170.05 99.3) (end 175.3 99.3) (width 0.2) (layer "F.Cu") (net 49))
 (segment (start 177.651 98.739058) (end 177.651 96.949) (width 0.2) (layer "F.Cu") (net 49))
 (segment (start 190.14 88.56) (end 191.66 88.56) (width 0.2) (layer "F.Cu") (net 49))
 (segment (start 175.454971 99.145029) (end 175.510942 99.201) (width 0.2) (layer "F.Cu") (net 49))
 (segment (start 184.6 90) (end 186.451 88.149) (width 0.2) (layer "F.Cu") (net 49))
 (segment (start 188 86.057164) (end 188 86.5) (width 0.2) (layer "F.Cu") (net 49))
 (segment (start 189.640001 88.56) (end 190.14 88.56) (width 0.2) (layer "F.Cu") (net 49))
 (segment (start 177.189058 99.201) (end 177.651 98.739058) (width 0.2) (layer "F.Cu") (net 49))
 (segment (start 186.451 88.149) (end 189.229001 88.149) (width 0.2) (layer "F.Cu") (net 49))
 (segment (start 175.510942 99.201) (end 177.189058 99.201) (width 0.2) (layer "F.Cu") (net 49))
 (segment (start 190.14 84.61) (end 191.66 84.61) (width 0.2) (layer "F.Cu") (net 49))
 (via (at 188 86.5) (size 0.6) (drill 0.3) (layers "F.Cu" "B.Cu") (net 49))
 (via (at 184.6 90) (size 0.6) (drill 0.3) (layers "F.Cu" "B.Cu") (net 49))
 (segment (start 188 86.9) (end 189.2 88.1) (width 0.2) (layer "B.Cu") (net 49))
 (segment (start 188 86.5) (end 188 86.9) (width 0.2) (layer "B.Cu") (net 49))
 (segment (start 181.5 80.107824) (end 179.307824 80.107824) (width 0.2) (layer "F.Cu") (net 41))
 (segment (start 191.135 78.45) (end 191.135 78.9) (width 0.2) (layer "F.Cu") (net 41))
 (segment (start 175.7 76.5) (end 174.3 76.5) (width 0.2) (layer "F.Cu") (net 41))
 (segment (start 179.307824 80.107824) (end 175.7 76.5) (width 0.2) (layer "F.Cu") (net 41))
 (segment (start 173.3 77.5) (end 173.3875 77.5875) (width 0.2) (layer "F.Cu") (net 41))
 (segment (start 183.1125 83.4) (end 183.1125 81.720324) (width 0.2) (layer "F.Cu") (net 41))
 (segment (start 189.927176 80.107824) (end 181.5 80.107824) (width 0.2) (layer "F.Cu") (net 41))
 (segment (start 191.135 78.9) (end 189.927176 80.107824) (width 0.2) (layer "F.Cu") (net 41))
 (segment (start 174.3 76.5) (end 173.3 77.5) (width 0.2) (layer "F.Cu") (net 41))
 (segment (start 183.1125 81.720324) (end 181.5 80.107824) (width 0.2) (layer "F.Cu") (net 41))
 (segment (start 173.3875 77.5875) (end 173.3875 79.2875) (width 0.2) (layer "F.Cu") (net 41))
 (segment (start 181.3875 78.8) (end 182.294324 79.706824) (width 0.2) (layer "F.Cu") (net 42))
 (segment (start 182.294324 79.706824) (end 189.058176 79.706824) (width 0.2) (layer "F.Cu") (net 42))
 (segment (start 172.8875 77.3454) (end 172.8875 79.2875) (width 0.2) (layer "F.Cu") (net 42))
 (segment (start 181.3875 78.8) (end 178.4875 75.9) (width 0.2) (layer "F.Cu") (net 42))
 (segment (start 178.4875 75.9) (end 174.3329 75.9) (width 0.2) (layer "F.Cu") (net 42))
 (segment (start 189.058176 79.706824) (end 189.865 78.9) (width 0.2) (layer "F.Cu") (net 42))
 (segment (start 174.3329 75.9) (end 172.8875 77.3454) (width 0.2) (layer "F.Cu") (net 42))
 (segment (start 189.865 78.9) (end 189.865 78.45) (width 0.2) (layer "F.Cu") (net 42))
 (segment (start 175.8875 78.2875) (end 175.2 77.6) (width 0.2) (layer "F.Cu") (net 36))
 (segment (start 175.8875 79.2875) (end 175.8875 78.2875) (width 0.2) (layer "F.Cu") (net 36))
 (via (at 175.2 77.6) (size 0.6) (drill 0.3) (layers "F.Cu" "B.Cu") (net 36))
 (via (at 174.1 72.9) (size 0.6) (drill 0.3) (layers "F.Cu" "B.Cu") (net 36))
 (segment (start 174.1 72.9) (end 175.2 74) (width 0.2) (layer "B.Cu") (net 36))
 (segment (start 175.2 74) (end 175.2 77.6) (width 0.2) (layer "B.Cu") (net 36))
 (segment (start 189.990001 87.620001) (end 190.14 87.77) (width 0.2) (layer "F.Cu") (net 47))
 (segment (start 185.7569 88.276) (end 186.412899 87.620001) (width 0.2) (layer "F.Cu") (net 47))
 (segment (start 181.9635 88.276) (end 185.7569 88.276) (width 0.2) (layer "F.Cu") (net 47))
 (segment (start 181.1875 87.5) (end 181.9635 88.276) (width 0.2) (layer "F.Cu") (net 47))
 (segment (start 186.412899 87.620001) (end 189.990001 87.620001) (width 0.2) (layer "F.Cu") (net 47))
 (segment (start 193.751496 85.4) (end 191.66 85.4) (width 0.2) (layer "F.Cu") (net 48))
 (segment (start 182.751 95.776) (end 190.924 95.776) (width 0.2) (layer "F.Cu") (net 48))
 (segment (start 190.924 95.776) (end 195.2 91.5) (width 0.2) (layer "F.Cu") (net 48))
 (segment (start 195.2 86.848504) (end 193.751496 85.4) (width 0.2) (layer "F.Cu") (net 48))
 (segment (start 195.2 91.5) (end 195.2 86.848504) (width 0.2) (layer "F.Cu") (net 48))
 (segment (start 181.975 95) (end 182.751 95.776) (width 0.2) (layer "F.Cu") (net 48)))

